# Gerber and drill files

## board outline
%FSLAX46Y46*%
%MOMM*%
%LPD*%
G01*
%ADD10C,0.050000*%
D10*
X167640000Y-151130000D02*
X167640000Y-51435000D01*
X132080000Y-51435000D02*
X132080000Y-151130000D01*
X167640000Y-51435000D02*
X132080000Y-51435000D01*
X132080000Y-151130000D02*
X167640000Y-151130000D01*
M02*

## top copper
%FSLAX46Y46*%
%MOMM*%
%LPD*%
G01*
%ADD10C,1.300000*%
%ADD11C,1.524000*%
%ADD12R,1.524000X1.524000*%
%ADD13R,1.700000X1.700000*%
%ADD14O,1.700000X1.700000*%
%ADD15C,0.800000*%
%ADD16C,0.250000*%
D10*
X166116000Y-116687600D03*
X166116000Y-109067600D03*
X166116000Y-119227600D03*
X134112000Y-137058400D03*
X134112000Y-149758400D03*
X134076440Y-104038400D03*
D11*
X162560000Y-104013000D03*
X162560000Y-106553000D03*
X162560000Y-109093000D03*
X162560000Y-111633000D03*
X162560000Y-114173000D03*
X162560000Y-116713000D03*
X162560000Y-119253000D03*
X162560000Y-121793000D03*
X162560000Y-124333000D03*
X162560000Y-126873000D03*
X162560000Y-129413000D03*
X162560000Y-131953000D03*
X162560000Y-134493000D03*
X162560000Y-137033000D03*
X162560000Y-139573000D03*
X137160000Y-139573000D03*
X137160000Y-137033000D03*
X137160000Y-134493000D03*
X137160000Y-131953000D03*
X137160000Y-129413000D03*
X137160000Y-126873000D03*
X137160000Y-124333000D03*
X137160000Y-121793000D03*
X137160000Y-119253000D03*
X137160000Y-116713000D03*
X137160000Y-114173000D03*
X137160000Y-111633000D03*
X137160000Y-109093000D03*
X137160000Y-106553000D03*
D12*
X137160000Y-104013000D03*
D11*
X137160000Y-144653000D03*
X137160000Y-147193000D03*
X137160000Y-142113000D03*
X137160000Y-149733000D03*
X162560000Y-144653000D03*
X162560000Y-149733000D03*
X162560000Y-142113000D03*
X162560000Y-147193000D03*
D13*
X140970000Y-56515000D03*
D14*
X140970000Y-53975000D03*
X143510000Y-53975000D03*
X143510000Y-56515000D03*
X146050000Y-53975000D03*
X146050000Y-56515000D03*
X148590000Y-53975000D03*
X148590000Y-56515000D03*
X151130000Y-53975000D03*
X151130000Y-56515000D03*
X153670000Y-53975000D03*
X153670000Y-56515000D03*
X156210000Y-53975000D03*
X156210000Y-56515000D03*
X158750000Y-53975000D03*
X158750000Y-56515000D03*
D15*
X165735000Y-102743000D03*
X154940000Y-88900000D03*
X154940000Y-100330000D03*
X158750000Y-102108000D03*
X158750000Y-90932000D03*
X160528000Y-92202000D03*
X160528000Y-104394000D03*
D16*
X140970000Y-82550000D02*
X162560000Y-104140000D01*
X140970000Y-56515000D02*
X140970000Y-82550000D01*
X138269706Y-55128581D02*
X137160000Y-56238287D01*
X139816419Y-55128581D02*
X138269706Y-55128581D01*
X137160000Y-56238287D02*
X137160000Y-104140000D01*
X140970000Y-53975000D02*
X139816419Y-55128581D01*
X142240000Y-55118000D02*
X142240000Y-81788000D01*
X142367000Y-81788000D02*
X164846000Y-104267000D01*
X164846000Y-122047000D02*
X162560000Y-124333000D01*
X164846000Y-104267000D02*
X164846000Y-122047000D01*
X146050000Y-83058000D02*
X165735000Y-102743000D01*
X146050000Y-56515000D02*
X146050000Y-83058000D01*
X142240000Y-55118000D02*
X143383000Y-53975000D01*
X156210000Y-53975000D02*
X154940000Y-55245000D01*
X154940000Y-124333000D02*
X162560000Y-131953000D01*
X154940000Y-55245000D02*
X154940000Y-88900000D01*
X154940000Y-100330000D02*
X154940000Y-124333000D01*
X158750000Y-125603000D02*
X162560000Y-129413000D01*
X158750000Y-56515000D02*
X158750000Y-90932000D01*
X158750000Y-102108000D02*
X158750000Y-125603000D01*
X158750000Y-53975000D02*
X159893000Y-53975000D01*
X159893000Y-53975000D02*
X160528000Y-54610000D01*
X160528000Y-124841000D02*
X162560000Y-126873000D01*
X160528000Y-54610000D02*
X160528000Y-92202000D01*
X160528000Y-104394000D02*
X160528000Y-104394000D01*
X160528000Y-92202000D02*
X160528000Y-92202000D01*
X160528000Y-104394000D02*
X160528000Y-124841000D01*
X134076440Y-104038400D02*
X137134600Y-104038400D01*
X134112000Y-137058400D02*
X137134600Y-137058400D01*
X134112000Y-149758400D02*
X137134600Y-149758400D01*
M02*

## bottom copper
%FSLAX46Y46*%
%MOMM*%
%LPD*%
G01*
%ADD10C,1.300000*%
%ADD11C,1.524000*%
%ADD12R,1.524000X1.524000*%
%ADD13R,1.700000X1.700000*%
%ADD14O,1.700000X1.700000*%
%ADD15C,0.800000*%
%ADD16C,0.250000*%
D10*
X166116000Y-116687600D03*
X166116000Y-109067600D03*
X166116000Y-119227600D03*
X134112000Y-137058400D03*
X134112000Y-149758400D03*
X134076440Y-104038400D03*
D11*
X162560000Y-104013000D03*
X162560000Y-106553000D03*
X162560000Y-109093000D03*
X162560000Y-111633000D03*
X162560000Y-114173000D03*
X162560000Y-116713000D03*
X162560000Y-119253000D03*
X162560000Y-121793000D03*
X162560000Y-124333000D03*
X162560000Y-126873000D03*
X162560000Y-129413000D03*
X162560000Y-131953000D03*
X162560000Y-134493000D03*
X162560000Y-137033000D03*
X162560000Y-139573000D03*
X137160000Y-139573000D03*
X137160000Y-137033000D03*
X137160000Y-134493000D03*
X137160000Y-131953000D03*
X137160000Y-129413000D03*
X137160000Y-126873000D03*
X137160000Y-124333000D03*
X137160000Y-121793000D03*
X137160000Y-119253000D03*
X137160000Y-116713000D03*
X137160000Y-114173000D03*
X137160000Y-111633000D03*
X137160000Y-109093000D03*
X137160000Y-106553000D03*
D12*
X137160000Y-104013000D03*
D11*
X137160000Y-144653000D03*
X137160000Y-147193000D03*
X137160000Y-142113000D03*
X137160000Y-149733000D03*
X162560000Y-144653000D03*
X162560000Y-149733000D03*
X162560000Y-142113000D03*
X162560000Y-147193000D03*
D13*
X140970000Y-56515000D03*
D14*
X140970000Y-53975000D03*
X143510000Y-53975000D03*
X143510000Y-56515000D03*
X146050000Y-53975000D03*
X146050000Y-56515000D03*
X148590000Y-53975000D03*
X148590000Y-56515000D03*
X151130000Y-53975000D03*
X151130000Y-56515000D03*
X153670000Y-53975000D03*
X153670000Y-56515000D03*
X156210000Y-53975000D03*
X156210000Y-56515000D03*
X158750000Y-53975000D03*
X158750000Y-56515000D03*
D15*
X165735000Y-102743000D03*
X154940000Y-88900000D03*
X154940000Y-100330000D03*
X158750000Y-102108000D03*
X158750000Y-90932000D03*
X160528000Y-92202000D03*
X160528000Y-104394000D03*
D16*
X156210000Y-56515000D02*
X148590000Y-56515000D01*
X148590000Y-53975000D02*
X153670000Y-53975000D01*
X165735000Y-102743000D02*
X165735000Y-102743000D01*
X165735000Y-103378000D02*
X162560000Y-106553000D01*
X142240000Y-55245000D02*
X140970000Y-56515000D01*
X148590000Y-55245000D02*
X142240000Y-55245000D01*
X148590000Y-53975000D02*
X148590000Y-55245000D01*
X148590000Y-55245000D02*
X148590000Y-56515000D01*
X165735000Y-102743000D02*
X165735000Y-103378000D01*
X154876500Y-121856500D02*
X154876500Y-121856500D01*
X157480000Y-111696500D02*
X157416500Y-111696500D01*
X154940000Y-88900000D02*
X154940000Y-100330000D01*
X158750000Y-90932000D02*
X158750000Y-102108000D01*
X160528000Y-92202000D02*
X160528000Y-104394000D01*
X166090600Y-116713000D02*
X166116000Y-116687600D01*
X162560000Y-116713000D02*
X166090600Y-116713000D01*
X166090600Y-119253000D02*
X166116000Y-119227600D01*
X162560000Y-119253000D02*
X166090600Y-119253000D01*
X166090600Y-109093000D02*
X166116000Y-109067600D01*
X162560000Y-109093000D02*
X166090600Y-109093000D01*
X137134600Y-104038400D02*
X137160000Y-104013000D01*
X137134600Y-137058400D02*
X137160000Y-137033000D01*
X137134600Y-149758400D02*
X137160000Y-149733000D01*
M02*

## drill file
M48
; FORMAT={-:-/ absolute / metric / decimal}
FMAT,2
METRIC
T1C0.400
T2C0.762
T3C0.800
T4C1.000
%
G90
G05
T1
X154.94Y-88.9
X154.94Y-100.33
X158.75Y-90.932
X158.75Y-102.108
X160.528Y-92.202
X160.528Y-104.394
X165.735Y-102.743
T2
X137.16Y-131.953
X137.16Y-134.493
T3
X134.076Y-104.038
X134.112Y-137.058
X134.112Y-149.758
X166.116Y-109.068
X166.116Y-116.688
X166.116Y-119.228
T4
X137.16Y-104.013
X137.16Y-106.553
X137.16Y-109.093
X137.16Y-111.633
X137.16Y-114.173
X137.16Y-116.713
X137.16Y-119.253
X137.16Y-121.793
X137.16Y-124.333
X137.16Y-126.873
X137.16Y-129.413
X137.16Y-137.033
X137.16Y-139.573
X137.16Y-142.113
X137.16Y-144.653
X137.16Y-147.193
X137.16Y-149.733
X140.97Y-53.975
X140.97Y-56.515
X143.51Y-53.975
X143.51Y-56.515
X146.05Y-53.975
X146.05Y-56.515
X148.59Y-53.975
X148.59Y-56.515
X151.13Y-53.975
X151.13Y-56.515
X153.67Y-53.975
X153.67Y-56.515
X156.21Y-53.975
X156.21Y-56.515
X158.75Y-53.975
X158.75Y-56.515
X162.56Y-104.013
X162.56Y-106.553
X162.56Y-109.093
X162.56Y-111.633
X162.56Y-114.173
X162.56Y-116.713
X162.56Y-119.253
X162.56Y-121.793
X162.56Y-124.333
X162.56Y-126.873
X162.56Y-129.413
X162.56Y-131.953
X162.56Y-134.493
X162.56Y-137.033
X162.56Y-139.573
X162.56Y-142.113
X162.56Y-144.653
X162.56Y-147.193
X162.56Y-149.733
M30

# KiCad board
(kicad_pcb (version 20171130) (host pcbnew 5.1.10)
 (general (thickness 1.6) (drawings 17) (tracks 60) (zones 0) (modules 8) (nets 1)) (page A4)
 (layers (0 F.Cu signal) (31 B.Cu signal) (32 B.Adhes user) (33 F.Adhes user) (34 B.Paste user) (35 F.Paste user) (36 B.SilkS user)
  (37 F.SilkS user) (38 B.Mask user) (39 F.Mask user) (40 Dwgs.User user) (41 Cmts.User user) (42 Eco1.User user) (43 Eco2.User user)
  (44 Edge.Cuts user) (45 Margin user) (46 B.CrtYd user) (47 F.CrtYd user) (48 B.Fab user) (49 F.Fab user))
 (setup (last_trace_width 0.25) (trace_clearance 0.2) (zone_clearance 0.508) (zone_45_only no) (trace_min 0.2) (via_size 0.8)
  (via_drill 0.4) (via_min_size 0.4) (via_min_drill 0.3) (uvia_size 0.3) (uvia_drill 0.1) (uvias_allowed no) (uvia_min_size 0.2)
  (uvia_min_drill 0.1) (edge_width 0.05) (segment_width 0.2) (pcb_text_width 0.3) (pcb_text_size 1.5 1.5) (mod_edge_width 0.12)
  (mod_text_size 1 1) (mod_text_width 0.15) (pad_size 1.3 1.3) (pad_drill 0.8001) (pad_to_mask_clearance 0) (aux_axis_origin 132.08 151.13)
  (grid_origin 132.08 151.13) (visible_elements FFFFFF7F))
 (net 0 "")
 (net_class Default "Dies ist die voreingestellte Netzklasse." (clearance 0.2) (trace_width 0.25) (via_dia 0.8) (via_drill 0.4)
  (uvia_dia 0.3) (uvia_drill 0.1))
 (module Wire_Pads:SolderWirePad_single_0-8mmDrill (layer F.Cu) (at 166.116 116.6876)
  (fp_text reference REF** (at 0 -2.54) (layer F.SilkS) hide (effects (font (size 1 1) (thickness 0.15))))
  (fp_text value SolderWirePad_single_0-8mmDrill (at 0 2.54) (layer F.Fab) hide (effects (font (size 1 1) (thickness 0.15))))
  (pad 1 thru_hole circle (at 0 0) (size 1.3 1.3) (drill 0.8001) (layers *.Cu *.Mask)))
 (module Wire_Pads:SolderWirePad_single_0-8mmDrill (layer F.Cu) (at 166.116 109.0676)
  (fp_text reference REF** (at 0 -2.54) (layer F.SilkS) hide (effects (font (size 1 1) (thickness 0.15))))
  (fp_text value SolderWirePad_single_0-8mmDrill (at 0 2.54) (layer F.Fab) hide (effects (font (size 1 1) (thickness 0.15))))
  (pad 1 thru_hole circle (at 0 0) (size 1.3 1.3) (drill 0.8001) (layers *.Cu *.Mask)))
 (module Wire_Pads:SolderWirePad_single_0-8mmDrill (layer F.Cu) (at 166.116 119.2276)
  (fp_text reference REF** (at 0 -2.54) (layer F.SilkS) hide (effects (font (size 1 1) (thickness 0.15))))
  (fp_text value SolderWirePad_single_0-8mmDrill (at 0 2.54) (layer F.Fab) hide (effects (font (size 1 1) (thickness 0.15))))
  (pad 1 thru_hole circle (at 0 0) (size 1.3 1.3) (drill 0.8001) (layers *.Cu *.Mask)))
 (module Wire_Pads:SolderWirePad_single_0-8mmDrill (layer F.Cu) (at 134.112 137.0584)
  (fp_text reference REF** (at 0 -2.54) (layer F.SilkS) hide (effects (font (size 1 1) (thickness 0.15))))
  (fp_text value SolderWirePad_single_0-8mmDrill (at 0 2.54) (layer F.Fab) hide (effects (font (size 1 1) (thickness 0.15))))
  (pad 1 thru_hole circle (at 0 0) (size 1.3 1.3) (drill 0.8001) (layers *.Cu *.Mask)))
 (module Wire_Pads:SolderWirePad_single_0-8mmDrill (layer F.Cu) (at 134.112 149.7584)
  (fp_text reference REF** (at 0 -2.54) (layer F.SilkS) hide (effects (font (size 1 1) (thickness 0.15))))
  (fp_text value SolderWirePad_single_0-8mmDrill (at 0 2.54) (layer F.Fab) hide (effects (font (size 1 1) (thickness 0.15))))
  (pad 1 thru_hole circle (at 0 0) (size 1.3 1.3) (drill 0.8001) (layers *.Cu *.Mask)))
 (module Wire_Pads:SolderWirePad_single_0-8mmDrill (layer F.Cu) (at 134.07644 104.0384)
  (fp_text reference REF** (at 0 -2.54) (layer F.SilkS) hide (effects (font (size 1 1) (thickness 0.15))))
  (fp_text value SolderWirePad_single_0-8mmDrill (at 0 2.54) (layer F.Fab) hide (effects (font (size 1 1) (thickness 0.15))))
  (pad 1 thru_hole circle (at 0 0) (size 1.3 1.3) (drill 0.8001) (layers *.Cu *.Mask)))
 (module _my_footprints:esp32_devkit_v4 (layer F.Cu) (at 149.86 104.013)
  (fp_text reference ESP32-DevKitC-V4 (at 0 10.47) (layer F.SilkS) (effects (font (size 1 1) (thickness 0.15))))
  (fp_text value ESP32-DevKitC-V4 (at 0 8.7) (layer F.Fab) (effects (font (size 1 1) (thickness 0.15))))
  (pad GND thru_hole circle (at 12.7 0) (size 1.524 1.524) (drill 1) (layers *.Cu *.Mask))
  (pad 23 thru_hole circle (at 12.7 2.54) (size 1.524 1.524) (drill 1) (layers *.Cu *.Mask))
  (pad 22 thru_hole circle (at 12.7 5.08) (size 1.524 1.524) (drill 1) (layers *.Cu *.Mask))
  (pad TX thru_hole circle (at 12.7 7.62) (size 1.524 1.524) (drill 1) (layers *.Cu *.Mask))
  (pad RX thru_hole circle (at 12.7 10.16) (size 1.524 1.524) (drill 1) (layers *.Cu *.Mask))
  (pad 21 thru_hole circle (at 12.7 12.7) (size 1.524 1.524) (drill 1) (layers *.Cu *.Mask))
  (pad GND thru_hole circle (at 12.7 15.24) (size 1.524 1.524) (drill 1) (layers *.Cu *.Mask))
  (pad 19 thru_hole circle (at 12.7 17.78) (size 1.524 1.524) (drill 1) (layers *.Cu *.Mask))
  (pad 18 thru_hole circle (at 12.7 20.32) (size 1.524 1.524) (drill 1) (layers *.Cu *.Mask))
  (pad 5 thru_hole circle (at 12.7 22.86) (size 1.524 1.524) (drill 1) (layers *.Cu *.Mask))
  (pad 17 thru_hole circle (at 12.7 25.4) (size 1.524 1.524) (drill 1) (layers *.Cu *.Mask))
  (pad 16 thru_hole circle (at 12.7 27.94) (size 1.524 1.524) (drill 1) (layers *.Cu *.Mask))
  (pad 4 thru_hole circle (at 12.7 30.48) (size 1.524 1.524) (drill 1) (layers *.Cu *.Mask))
  (pad 0 thru_hole circle (at 12.7 33.02) (size 1.524 1.524) (drill 1) (layers *.Cu *.Mask))
  (pad 2 thru_hole circle (at 12.7 35.56) (size 1.524 1.524) (drill 1) (layers *.Cu *.Mask))
  (pad 13 thru_hole circle (at -12.7 35.56) (size 1.524 1.524) (drill 1) (layers *.Cu *.Mask))
  (pad GND thru_hole circle (at -12.7 33.02) (size 1.524 1.524) (drill 1) (layers *.Cu *.Mask))
  (pad 12 thru_hole circle (at -12.7 30.48) (size 1.524 1.524) (drill 0.762) (layers *.Cu *.Mask))
  (pad 14 thru_hole circle (at -12.7 27.94) (size 1.524 1.524) (drill 0.762) (layers *.Cu *.Mask))
  (pad 27 thru_hole circle (at -12.7 25.4) (size 1.524 1.524) (drill 1) (layers *.Cu *.Mask))
  (pad 26 thru_hole circle (at -12.7 22.86) (size 1.524 1.524) (drill 1) (layers *.Cu *.Mask))
  (pad 25 thru_hole circle (at -12.7 20.32) (size 1.524 1.524) (drill 1) (layers *.Cu *.Mask))
  (pad 33 thru_hole circle (at -12.7 17.78) (size 1.524 1.524) (drill 1) (layers *.Cu *.Mask))
  (pad 32 thru_hole circle (at -12.7 15.24) (size 1.524 1.524) (drill 1) (layers *.Cu *.Mask))
  (pad 35 thru_hole circle (at -12.7 12.7) (size 1.524 1.524) (drill 1) (layers *.Cu *.Mask))
  (pad 34 thru_hole circle (at -12.7 10.16) (size 1.524 1.524) (drill 1) (layers *.Cu *.Mask))
  (pad VN thru_hole circle (at -12.7 7.62) (size 1.524 1.524) (drill 1) (layers *.Cu *.Mask))
  (pad VP thru_hole circle (at -12.7 5.08) (size 1.524 1.524) (drill 1) (layers *.Cu *.Mask))
  (pad CN thru_hole circle (at -12.7 2.54) (size 1.524 1.524) (drill 1) (layers *.Cu *.Mask))
  (pad 3V3 thru_hole rect (at -12.7 0) (size 1.524 1.524) (drill 1) (layers *.Cu *.Mask))
  (pad D3 thru_hole circle (at -12.7 40.64) (size 1.524 1.524) (drill 1) (layers *.Cu *.Mask))
  (pad CMD thru_hole circle (at -12.7 43.18) (size 1.524 1.524) (drill 1) (layers *.Cu *.Mask))
  (pad D2 thru_hole circle (at -12.7 38.1) (size 1.524 1.524) (drill 1) (layers *.Cu *.Mask))
  (pad 5V thru_hole circle (at -12.7 45.72) (size 1.524 1.524) (drill 1) (layers *.Cu *.Mask))
  (pad D1 thru_hole circle (at 12.7 40.64) (size 1.524 1.524) (drill 1) (layers *.Cu *.Mask))
  (pad CLK thru_hole circle (at 12.7 45.72) (size 1.524 1.524) (drill 1) (layers *.Cu *.Mask))
  (pad 15 thru_hole circle (at 12.7 38.1) (size 1.524 1.524) (drill 1) (layers *.Cu *.Mask))
  (pad D0 thru_hole circle (at 12.7 43.18) (size 1.524 1.524) (drill 1) (layers *.Cu *.Mask)))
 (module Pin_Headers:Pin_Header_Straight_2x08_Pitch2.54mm (layer B.Cu) (at 140.97 53.975 270)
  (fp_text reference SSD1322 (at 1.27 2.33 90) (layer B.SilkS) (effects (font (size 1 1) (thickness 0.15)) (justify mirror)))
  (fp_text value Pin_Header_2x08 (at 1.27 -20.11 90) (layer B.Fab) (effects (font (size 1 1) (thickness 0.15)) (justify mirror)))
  (pad 1 thru_hole rect (at 2.54 0 270) (size 1.7 1.7) (drill 1) (layers *.Cu *.Mask))
  (pad 2 thru_hole oval (at 0 0 270) (size 1.7 1.7) (drill 1) (layers *.Cu *.Mask))
  (pad 4 thru_hole oval (at 0 -2.54 270) (size 1.7 1.7) (drill 1) (layers *.Cu *.Mask))
  (pad 3 thru_hole oval (at 2.54 -2.54 270) (size 1.7 1.7) (drill 1) (layers *.Cu *.Mask))
  (pad 6 thru_hole oval (at 0 -5.08 270) (size 1.7 1.7) (drill 1) (layers *.Cu *.Mask))
  (pad 5 thru_hole oval (at 2.54 -5.08 270) (size 1.7 1.7) (drill 1) (layers *.Cu *.Mask))
  (pad 8 thru_hole oval (at 0 -7.62 270) (size 1.7 1.7) (drill 1) (layers *.Cu *.Mask))
  (pad 7 thru_hole oval (at 2.54 -7.62 270) (size 1.7 1.7) (drill 1) (layers *.Cu *.Mask))
  (pad 10 thru_hole oval (at 0 -10.16 270) (size 1.7 1.7) (drill 1) (layers *.Cu *.Mask))
  (pad 9 thru_hole oval (at 2.54 -10.16 270) (size 1.7 1.7) (drill 1) (layers *.Cu *.Mask))
  (pad 12 thru_hole oval (at 0 -12.7 270) (size 1.7 1.7) (drill 1) (layers *.Cu *.Mask))
  (pad 11 thru_hole oval (at 2.54 -12.7 270) (size 1.7 1.7) (drill 1) (layers *.Cu *.Mask))
  (pad 14 thru_hole oval (at 0 -15.24 270) (size 1.7 1.7) (drill 1) (layers *.Cu *.Mask))
  (pad 13 thru_hole oval (at 2.54 -15.24 270) (size 1.7 1.7) (drill 1) (layers *.Cu *.Mask))
  (pad 16 thru_hole oval (at 0 -17.78 270) (size 1.7 1.7) (drill 1) (layers *.Cu *.Mask))
  (pad 15 thru_hole oval (at 2.54 -17.78 270) (size 1.7 1.7) (drill 1) (layers *.Cu *.Mask)))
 (gr_line (start 167.64 151.13) (end 167.64 51.435) (layer Edge.Cuts) (width 0.05))
 (gr_line (start 132.08 51.435) (end 132.08 151.13) (layer Edge.Cuts) (width 0.05))
 (gr_line (start 167.64 51.435) (end 132.08 51.435) (layer Edge.Cuts) (width 0.05))
 (gr_line (start 132.08 151.13) (end 167.64 151.13) (layer Edge.Cuts) (width 0.05))
 (segment (start 156.21 56.515) (end 148.59 56.515) (width 0.25) (layer B.Cu) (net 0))
 (segment (start 148.59 53.975) (end 153.67 53.975) (width 0.25) (layer B.Cu) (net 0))
 (segment (start 140.97 82.55) (end 162.56 104.14) (width 0.25) (layer F.Cu) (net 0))
 (segment (start 140.97 56.515) (end 140.97 82.55) (width 0.25) (layer F.Cu) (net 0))
 (segment (start 138.269706 55.128581) (end 137.16 56.238287) (width 0.25) (layer F.Cu) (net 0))
 (segment (start 139.816419 55.128581) (end 138.269706 55.128581) (width 0.25) (layer F.Cu) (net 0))
 (segment (start 137.16 56.238287) (end 137.16 104.14) (width 0.25) (layer F.Cu) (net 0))
 (segment (start 140.97 53.975) (end 139.816419 55.128581) (width 0.25) (layer F.Cu) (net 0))
 (segment (start 142.24 55.118) (end 142.24 81.788) (width 0.25) (layer F.Cu) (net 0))
 (segment (start 142.367 81.788) (end 164.846 104.267) (width 0.25) (layer F.Cu) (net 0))
 (segment (start 164.846 122.047) (end 162.56 124.333) (width 0.25) (layer F.Cu) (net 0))
 (segment (start 164.846 104.267) (end 164.846 122.047) (width 0.25) (layer F.Cu) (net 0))
 (segment (start 165.735 102.743) (end 165.735 102.743) (width 0.25) (layer B.Cu) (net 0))
 (segment (start 165.735 103.378) (end 162.56 106.553) (width 0.25) (layer B.Cu) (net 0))
 (segment (start 146.05 83.058) (end 165.735 102.743) (width 0.25) (layer F.Cu) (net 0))
 (segment (start 146.05 56.515) (end 146.05 83.058) (width 0.25) (layer F.Cu) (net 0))
 (segment (start 142.24 55.245) (end 140.97 56.515) (width 0.25) (layer B.Cu) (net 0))
 (segment (start 148.59 55.245) (end 142.24 55.245) (width 0.25) (layer B.Cu) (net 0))
 (segment (start 148.59 53.975) (end 148.59 55.245) (width 0.25) (layer B.Cu) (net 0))
 (segment (start 148.59 55.245) (end 148.59 56.515) (width 0.25) (layer B.Cu) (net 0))
 (segment (start 165.735 102.743) (end 165.735 103.378) (width 0.25) (layer B.Cu) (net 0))
 (via (at 165.735 102.743) (size 0.8) (drill 0.4) (layers F.Cu B.Cu) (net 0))
 (segment (start 154.8765 121.8565) (end 154.8765 121.8565) (width 0.25) (layer B.Cu) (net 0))
 (segment (start 157.48 111.6965) (end 157.4165 111.6965) (width 0.25) (layer B.Cu) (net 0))
 (segment (start 142.24 55.118) (end 143.383 53.975) (width 0.25) (layer F.Cu) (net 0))
 (segment (start 156.21 53.975) (end 154.94 55.245) (width 0.25) (layer F.Cu) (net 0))
 (segment (start 154.94 124.333) (end 162.56 131.953) (width 0.25) (layer F.Cu) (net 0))
 (segment (start 154.94 55.245) (end 154.94 88.9) (width 0.25) (layer F.Cu) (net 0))
 (segment (start 154.94 88.9) (end 154.94 100.33) (width 0.25) (layer B.Cu) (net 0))
 (via (at 154.94 88.9) (size 0.8) (drill 0.4) (layers F.Cu B.Cu) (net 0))
 (segment (start 154.94 100.33) (end 154.94 124.333) (width 0.25) (layer F.Cu) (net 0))
 (via (at 154.94 100.33) (size 0.8) (drill 0.4) (layers F.Cu B.Cu) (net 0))
 (segment (start 158.75 125.603) (end 162.56 129.413) (width 0.25) (layer F.Cu) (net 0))
 (segment (start 158.75 56.515) (end 158.75 90.932) (width 0.25) (layer F.Cu) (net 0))
 (segment (start 158.75 102.108) (end 158.75 125.603) (width 0.25) (layer F.Cu) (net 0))
 (via (at 158.75 102.108) (size 0.8) (drill 0.4) (layers F.Cu B.Cu) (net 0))
 (segment (start 158.75 90.932) (end 158.75 102.108) (width 0.25) (layer B.Cu) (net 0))
 (via (at 158.75 90.932) (size 0.8) (drill 0.4) (layers F.Cu B.Cu) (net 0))
 (segment (start 158.75 53.975) (end 159.893 53.975) (width 0.25) (layer F.Cu) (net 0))
 (segment (start 159.893 53.975) (end 160.528 54.61) (width 0.25) (layer F.Cu) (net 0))
 (segment (start 160.528 124.841) (end 162.56 126.873) (width 0.25) (layer F.Cu) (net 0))
 (segment (start 160.528 54.61) (end 160.528 92.202) (width 0.25) (layer F.Cu) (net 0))
 (segment (start 160.528 92.202) (end 160.528 104.394) (width 0.25) (layer B.Cu) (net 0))
 (segment (start 160.528 104.394) (end 160.528 104.394) (width 0.25) (layer F.Cu) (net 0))
 (segment (start 160.528 92.202) (end 160.528 92.202) (width 0.25) (layer F.Cu) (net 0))
 (via (at 160.528 92.202) (size 0.8) (drill 0.4) (layers F.Cu B.Cu) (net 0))
 (segment (start 160.528 104.394) (end 160.528 124.841) (width 0.25) (layer F.Cu) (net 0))
 (via (at 160.528 104.394) (size 0.8) (drill 0.4) (layers F.Cu B.Cu) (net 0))
 (segment (start 166.0906 116.713) (end 166.116 116.6876) (width 0.25) (layer B.Cu) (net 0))
 (segment (start 162.56 116.713) (end 166.0906 116.713) (width 0.25) (layer B.Cu) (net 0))
 (segment (start 166.0906 119.253) (end 166.116 119.2276) (width 0.25) (layer B.Cu) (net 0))
 (segment (start 162.56 119.253) (end 166.0906 119.253) (width 0.25) (layer B.Cu) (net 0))
 (segment (start 166.0906 109.093) (end 166.116 109.0676) (width 0.25) (layer B.Cu) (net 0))
 (segment (start 162.56 109.093) (end 166.0906 109.093) (width 0.25) (layer B.Cu) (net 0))
 (segment (start 137.1346 104.0384) (end 137.16 104.013) (width 0.25) (layer B.Cu) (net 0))
 (segment (start 134.07644 104.0384) (end 137.1346 104.0384) (width 0.25) (layer F.Cu) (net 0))
 (segment (start 137.1346 137.0584) (end 137.16 137.033) (width 0.25) (layer B.Cu) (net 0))
 (segment (start 134.112 137.0584) (end 137.1346 137.0584) (width 0.25) (layer F.Cu) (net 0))
 (segment (start 137.1346 149.7584) (end 137.16 149.733) (width 0.25) (layer B.Cu) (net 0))
 (segment (start 134.112 149.7584) (end 137.1346 149.7584) (width 0.25) (layer F.Cu) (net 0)))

